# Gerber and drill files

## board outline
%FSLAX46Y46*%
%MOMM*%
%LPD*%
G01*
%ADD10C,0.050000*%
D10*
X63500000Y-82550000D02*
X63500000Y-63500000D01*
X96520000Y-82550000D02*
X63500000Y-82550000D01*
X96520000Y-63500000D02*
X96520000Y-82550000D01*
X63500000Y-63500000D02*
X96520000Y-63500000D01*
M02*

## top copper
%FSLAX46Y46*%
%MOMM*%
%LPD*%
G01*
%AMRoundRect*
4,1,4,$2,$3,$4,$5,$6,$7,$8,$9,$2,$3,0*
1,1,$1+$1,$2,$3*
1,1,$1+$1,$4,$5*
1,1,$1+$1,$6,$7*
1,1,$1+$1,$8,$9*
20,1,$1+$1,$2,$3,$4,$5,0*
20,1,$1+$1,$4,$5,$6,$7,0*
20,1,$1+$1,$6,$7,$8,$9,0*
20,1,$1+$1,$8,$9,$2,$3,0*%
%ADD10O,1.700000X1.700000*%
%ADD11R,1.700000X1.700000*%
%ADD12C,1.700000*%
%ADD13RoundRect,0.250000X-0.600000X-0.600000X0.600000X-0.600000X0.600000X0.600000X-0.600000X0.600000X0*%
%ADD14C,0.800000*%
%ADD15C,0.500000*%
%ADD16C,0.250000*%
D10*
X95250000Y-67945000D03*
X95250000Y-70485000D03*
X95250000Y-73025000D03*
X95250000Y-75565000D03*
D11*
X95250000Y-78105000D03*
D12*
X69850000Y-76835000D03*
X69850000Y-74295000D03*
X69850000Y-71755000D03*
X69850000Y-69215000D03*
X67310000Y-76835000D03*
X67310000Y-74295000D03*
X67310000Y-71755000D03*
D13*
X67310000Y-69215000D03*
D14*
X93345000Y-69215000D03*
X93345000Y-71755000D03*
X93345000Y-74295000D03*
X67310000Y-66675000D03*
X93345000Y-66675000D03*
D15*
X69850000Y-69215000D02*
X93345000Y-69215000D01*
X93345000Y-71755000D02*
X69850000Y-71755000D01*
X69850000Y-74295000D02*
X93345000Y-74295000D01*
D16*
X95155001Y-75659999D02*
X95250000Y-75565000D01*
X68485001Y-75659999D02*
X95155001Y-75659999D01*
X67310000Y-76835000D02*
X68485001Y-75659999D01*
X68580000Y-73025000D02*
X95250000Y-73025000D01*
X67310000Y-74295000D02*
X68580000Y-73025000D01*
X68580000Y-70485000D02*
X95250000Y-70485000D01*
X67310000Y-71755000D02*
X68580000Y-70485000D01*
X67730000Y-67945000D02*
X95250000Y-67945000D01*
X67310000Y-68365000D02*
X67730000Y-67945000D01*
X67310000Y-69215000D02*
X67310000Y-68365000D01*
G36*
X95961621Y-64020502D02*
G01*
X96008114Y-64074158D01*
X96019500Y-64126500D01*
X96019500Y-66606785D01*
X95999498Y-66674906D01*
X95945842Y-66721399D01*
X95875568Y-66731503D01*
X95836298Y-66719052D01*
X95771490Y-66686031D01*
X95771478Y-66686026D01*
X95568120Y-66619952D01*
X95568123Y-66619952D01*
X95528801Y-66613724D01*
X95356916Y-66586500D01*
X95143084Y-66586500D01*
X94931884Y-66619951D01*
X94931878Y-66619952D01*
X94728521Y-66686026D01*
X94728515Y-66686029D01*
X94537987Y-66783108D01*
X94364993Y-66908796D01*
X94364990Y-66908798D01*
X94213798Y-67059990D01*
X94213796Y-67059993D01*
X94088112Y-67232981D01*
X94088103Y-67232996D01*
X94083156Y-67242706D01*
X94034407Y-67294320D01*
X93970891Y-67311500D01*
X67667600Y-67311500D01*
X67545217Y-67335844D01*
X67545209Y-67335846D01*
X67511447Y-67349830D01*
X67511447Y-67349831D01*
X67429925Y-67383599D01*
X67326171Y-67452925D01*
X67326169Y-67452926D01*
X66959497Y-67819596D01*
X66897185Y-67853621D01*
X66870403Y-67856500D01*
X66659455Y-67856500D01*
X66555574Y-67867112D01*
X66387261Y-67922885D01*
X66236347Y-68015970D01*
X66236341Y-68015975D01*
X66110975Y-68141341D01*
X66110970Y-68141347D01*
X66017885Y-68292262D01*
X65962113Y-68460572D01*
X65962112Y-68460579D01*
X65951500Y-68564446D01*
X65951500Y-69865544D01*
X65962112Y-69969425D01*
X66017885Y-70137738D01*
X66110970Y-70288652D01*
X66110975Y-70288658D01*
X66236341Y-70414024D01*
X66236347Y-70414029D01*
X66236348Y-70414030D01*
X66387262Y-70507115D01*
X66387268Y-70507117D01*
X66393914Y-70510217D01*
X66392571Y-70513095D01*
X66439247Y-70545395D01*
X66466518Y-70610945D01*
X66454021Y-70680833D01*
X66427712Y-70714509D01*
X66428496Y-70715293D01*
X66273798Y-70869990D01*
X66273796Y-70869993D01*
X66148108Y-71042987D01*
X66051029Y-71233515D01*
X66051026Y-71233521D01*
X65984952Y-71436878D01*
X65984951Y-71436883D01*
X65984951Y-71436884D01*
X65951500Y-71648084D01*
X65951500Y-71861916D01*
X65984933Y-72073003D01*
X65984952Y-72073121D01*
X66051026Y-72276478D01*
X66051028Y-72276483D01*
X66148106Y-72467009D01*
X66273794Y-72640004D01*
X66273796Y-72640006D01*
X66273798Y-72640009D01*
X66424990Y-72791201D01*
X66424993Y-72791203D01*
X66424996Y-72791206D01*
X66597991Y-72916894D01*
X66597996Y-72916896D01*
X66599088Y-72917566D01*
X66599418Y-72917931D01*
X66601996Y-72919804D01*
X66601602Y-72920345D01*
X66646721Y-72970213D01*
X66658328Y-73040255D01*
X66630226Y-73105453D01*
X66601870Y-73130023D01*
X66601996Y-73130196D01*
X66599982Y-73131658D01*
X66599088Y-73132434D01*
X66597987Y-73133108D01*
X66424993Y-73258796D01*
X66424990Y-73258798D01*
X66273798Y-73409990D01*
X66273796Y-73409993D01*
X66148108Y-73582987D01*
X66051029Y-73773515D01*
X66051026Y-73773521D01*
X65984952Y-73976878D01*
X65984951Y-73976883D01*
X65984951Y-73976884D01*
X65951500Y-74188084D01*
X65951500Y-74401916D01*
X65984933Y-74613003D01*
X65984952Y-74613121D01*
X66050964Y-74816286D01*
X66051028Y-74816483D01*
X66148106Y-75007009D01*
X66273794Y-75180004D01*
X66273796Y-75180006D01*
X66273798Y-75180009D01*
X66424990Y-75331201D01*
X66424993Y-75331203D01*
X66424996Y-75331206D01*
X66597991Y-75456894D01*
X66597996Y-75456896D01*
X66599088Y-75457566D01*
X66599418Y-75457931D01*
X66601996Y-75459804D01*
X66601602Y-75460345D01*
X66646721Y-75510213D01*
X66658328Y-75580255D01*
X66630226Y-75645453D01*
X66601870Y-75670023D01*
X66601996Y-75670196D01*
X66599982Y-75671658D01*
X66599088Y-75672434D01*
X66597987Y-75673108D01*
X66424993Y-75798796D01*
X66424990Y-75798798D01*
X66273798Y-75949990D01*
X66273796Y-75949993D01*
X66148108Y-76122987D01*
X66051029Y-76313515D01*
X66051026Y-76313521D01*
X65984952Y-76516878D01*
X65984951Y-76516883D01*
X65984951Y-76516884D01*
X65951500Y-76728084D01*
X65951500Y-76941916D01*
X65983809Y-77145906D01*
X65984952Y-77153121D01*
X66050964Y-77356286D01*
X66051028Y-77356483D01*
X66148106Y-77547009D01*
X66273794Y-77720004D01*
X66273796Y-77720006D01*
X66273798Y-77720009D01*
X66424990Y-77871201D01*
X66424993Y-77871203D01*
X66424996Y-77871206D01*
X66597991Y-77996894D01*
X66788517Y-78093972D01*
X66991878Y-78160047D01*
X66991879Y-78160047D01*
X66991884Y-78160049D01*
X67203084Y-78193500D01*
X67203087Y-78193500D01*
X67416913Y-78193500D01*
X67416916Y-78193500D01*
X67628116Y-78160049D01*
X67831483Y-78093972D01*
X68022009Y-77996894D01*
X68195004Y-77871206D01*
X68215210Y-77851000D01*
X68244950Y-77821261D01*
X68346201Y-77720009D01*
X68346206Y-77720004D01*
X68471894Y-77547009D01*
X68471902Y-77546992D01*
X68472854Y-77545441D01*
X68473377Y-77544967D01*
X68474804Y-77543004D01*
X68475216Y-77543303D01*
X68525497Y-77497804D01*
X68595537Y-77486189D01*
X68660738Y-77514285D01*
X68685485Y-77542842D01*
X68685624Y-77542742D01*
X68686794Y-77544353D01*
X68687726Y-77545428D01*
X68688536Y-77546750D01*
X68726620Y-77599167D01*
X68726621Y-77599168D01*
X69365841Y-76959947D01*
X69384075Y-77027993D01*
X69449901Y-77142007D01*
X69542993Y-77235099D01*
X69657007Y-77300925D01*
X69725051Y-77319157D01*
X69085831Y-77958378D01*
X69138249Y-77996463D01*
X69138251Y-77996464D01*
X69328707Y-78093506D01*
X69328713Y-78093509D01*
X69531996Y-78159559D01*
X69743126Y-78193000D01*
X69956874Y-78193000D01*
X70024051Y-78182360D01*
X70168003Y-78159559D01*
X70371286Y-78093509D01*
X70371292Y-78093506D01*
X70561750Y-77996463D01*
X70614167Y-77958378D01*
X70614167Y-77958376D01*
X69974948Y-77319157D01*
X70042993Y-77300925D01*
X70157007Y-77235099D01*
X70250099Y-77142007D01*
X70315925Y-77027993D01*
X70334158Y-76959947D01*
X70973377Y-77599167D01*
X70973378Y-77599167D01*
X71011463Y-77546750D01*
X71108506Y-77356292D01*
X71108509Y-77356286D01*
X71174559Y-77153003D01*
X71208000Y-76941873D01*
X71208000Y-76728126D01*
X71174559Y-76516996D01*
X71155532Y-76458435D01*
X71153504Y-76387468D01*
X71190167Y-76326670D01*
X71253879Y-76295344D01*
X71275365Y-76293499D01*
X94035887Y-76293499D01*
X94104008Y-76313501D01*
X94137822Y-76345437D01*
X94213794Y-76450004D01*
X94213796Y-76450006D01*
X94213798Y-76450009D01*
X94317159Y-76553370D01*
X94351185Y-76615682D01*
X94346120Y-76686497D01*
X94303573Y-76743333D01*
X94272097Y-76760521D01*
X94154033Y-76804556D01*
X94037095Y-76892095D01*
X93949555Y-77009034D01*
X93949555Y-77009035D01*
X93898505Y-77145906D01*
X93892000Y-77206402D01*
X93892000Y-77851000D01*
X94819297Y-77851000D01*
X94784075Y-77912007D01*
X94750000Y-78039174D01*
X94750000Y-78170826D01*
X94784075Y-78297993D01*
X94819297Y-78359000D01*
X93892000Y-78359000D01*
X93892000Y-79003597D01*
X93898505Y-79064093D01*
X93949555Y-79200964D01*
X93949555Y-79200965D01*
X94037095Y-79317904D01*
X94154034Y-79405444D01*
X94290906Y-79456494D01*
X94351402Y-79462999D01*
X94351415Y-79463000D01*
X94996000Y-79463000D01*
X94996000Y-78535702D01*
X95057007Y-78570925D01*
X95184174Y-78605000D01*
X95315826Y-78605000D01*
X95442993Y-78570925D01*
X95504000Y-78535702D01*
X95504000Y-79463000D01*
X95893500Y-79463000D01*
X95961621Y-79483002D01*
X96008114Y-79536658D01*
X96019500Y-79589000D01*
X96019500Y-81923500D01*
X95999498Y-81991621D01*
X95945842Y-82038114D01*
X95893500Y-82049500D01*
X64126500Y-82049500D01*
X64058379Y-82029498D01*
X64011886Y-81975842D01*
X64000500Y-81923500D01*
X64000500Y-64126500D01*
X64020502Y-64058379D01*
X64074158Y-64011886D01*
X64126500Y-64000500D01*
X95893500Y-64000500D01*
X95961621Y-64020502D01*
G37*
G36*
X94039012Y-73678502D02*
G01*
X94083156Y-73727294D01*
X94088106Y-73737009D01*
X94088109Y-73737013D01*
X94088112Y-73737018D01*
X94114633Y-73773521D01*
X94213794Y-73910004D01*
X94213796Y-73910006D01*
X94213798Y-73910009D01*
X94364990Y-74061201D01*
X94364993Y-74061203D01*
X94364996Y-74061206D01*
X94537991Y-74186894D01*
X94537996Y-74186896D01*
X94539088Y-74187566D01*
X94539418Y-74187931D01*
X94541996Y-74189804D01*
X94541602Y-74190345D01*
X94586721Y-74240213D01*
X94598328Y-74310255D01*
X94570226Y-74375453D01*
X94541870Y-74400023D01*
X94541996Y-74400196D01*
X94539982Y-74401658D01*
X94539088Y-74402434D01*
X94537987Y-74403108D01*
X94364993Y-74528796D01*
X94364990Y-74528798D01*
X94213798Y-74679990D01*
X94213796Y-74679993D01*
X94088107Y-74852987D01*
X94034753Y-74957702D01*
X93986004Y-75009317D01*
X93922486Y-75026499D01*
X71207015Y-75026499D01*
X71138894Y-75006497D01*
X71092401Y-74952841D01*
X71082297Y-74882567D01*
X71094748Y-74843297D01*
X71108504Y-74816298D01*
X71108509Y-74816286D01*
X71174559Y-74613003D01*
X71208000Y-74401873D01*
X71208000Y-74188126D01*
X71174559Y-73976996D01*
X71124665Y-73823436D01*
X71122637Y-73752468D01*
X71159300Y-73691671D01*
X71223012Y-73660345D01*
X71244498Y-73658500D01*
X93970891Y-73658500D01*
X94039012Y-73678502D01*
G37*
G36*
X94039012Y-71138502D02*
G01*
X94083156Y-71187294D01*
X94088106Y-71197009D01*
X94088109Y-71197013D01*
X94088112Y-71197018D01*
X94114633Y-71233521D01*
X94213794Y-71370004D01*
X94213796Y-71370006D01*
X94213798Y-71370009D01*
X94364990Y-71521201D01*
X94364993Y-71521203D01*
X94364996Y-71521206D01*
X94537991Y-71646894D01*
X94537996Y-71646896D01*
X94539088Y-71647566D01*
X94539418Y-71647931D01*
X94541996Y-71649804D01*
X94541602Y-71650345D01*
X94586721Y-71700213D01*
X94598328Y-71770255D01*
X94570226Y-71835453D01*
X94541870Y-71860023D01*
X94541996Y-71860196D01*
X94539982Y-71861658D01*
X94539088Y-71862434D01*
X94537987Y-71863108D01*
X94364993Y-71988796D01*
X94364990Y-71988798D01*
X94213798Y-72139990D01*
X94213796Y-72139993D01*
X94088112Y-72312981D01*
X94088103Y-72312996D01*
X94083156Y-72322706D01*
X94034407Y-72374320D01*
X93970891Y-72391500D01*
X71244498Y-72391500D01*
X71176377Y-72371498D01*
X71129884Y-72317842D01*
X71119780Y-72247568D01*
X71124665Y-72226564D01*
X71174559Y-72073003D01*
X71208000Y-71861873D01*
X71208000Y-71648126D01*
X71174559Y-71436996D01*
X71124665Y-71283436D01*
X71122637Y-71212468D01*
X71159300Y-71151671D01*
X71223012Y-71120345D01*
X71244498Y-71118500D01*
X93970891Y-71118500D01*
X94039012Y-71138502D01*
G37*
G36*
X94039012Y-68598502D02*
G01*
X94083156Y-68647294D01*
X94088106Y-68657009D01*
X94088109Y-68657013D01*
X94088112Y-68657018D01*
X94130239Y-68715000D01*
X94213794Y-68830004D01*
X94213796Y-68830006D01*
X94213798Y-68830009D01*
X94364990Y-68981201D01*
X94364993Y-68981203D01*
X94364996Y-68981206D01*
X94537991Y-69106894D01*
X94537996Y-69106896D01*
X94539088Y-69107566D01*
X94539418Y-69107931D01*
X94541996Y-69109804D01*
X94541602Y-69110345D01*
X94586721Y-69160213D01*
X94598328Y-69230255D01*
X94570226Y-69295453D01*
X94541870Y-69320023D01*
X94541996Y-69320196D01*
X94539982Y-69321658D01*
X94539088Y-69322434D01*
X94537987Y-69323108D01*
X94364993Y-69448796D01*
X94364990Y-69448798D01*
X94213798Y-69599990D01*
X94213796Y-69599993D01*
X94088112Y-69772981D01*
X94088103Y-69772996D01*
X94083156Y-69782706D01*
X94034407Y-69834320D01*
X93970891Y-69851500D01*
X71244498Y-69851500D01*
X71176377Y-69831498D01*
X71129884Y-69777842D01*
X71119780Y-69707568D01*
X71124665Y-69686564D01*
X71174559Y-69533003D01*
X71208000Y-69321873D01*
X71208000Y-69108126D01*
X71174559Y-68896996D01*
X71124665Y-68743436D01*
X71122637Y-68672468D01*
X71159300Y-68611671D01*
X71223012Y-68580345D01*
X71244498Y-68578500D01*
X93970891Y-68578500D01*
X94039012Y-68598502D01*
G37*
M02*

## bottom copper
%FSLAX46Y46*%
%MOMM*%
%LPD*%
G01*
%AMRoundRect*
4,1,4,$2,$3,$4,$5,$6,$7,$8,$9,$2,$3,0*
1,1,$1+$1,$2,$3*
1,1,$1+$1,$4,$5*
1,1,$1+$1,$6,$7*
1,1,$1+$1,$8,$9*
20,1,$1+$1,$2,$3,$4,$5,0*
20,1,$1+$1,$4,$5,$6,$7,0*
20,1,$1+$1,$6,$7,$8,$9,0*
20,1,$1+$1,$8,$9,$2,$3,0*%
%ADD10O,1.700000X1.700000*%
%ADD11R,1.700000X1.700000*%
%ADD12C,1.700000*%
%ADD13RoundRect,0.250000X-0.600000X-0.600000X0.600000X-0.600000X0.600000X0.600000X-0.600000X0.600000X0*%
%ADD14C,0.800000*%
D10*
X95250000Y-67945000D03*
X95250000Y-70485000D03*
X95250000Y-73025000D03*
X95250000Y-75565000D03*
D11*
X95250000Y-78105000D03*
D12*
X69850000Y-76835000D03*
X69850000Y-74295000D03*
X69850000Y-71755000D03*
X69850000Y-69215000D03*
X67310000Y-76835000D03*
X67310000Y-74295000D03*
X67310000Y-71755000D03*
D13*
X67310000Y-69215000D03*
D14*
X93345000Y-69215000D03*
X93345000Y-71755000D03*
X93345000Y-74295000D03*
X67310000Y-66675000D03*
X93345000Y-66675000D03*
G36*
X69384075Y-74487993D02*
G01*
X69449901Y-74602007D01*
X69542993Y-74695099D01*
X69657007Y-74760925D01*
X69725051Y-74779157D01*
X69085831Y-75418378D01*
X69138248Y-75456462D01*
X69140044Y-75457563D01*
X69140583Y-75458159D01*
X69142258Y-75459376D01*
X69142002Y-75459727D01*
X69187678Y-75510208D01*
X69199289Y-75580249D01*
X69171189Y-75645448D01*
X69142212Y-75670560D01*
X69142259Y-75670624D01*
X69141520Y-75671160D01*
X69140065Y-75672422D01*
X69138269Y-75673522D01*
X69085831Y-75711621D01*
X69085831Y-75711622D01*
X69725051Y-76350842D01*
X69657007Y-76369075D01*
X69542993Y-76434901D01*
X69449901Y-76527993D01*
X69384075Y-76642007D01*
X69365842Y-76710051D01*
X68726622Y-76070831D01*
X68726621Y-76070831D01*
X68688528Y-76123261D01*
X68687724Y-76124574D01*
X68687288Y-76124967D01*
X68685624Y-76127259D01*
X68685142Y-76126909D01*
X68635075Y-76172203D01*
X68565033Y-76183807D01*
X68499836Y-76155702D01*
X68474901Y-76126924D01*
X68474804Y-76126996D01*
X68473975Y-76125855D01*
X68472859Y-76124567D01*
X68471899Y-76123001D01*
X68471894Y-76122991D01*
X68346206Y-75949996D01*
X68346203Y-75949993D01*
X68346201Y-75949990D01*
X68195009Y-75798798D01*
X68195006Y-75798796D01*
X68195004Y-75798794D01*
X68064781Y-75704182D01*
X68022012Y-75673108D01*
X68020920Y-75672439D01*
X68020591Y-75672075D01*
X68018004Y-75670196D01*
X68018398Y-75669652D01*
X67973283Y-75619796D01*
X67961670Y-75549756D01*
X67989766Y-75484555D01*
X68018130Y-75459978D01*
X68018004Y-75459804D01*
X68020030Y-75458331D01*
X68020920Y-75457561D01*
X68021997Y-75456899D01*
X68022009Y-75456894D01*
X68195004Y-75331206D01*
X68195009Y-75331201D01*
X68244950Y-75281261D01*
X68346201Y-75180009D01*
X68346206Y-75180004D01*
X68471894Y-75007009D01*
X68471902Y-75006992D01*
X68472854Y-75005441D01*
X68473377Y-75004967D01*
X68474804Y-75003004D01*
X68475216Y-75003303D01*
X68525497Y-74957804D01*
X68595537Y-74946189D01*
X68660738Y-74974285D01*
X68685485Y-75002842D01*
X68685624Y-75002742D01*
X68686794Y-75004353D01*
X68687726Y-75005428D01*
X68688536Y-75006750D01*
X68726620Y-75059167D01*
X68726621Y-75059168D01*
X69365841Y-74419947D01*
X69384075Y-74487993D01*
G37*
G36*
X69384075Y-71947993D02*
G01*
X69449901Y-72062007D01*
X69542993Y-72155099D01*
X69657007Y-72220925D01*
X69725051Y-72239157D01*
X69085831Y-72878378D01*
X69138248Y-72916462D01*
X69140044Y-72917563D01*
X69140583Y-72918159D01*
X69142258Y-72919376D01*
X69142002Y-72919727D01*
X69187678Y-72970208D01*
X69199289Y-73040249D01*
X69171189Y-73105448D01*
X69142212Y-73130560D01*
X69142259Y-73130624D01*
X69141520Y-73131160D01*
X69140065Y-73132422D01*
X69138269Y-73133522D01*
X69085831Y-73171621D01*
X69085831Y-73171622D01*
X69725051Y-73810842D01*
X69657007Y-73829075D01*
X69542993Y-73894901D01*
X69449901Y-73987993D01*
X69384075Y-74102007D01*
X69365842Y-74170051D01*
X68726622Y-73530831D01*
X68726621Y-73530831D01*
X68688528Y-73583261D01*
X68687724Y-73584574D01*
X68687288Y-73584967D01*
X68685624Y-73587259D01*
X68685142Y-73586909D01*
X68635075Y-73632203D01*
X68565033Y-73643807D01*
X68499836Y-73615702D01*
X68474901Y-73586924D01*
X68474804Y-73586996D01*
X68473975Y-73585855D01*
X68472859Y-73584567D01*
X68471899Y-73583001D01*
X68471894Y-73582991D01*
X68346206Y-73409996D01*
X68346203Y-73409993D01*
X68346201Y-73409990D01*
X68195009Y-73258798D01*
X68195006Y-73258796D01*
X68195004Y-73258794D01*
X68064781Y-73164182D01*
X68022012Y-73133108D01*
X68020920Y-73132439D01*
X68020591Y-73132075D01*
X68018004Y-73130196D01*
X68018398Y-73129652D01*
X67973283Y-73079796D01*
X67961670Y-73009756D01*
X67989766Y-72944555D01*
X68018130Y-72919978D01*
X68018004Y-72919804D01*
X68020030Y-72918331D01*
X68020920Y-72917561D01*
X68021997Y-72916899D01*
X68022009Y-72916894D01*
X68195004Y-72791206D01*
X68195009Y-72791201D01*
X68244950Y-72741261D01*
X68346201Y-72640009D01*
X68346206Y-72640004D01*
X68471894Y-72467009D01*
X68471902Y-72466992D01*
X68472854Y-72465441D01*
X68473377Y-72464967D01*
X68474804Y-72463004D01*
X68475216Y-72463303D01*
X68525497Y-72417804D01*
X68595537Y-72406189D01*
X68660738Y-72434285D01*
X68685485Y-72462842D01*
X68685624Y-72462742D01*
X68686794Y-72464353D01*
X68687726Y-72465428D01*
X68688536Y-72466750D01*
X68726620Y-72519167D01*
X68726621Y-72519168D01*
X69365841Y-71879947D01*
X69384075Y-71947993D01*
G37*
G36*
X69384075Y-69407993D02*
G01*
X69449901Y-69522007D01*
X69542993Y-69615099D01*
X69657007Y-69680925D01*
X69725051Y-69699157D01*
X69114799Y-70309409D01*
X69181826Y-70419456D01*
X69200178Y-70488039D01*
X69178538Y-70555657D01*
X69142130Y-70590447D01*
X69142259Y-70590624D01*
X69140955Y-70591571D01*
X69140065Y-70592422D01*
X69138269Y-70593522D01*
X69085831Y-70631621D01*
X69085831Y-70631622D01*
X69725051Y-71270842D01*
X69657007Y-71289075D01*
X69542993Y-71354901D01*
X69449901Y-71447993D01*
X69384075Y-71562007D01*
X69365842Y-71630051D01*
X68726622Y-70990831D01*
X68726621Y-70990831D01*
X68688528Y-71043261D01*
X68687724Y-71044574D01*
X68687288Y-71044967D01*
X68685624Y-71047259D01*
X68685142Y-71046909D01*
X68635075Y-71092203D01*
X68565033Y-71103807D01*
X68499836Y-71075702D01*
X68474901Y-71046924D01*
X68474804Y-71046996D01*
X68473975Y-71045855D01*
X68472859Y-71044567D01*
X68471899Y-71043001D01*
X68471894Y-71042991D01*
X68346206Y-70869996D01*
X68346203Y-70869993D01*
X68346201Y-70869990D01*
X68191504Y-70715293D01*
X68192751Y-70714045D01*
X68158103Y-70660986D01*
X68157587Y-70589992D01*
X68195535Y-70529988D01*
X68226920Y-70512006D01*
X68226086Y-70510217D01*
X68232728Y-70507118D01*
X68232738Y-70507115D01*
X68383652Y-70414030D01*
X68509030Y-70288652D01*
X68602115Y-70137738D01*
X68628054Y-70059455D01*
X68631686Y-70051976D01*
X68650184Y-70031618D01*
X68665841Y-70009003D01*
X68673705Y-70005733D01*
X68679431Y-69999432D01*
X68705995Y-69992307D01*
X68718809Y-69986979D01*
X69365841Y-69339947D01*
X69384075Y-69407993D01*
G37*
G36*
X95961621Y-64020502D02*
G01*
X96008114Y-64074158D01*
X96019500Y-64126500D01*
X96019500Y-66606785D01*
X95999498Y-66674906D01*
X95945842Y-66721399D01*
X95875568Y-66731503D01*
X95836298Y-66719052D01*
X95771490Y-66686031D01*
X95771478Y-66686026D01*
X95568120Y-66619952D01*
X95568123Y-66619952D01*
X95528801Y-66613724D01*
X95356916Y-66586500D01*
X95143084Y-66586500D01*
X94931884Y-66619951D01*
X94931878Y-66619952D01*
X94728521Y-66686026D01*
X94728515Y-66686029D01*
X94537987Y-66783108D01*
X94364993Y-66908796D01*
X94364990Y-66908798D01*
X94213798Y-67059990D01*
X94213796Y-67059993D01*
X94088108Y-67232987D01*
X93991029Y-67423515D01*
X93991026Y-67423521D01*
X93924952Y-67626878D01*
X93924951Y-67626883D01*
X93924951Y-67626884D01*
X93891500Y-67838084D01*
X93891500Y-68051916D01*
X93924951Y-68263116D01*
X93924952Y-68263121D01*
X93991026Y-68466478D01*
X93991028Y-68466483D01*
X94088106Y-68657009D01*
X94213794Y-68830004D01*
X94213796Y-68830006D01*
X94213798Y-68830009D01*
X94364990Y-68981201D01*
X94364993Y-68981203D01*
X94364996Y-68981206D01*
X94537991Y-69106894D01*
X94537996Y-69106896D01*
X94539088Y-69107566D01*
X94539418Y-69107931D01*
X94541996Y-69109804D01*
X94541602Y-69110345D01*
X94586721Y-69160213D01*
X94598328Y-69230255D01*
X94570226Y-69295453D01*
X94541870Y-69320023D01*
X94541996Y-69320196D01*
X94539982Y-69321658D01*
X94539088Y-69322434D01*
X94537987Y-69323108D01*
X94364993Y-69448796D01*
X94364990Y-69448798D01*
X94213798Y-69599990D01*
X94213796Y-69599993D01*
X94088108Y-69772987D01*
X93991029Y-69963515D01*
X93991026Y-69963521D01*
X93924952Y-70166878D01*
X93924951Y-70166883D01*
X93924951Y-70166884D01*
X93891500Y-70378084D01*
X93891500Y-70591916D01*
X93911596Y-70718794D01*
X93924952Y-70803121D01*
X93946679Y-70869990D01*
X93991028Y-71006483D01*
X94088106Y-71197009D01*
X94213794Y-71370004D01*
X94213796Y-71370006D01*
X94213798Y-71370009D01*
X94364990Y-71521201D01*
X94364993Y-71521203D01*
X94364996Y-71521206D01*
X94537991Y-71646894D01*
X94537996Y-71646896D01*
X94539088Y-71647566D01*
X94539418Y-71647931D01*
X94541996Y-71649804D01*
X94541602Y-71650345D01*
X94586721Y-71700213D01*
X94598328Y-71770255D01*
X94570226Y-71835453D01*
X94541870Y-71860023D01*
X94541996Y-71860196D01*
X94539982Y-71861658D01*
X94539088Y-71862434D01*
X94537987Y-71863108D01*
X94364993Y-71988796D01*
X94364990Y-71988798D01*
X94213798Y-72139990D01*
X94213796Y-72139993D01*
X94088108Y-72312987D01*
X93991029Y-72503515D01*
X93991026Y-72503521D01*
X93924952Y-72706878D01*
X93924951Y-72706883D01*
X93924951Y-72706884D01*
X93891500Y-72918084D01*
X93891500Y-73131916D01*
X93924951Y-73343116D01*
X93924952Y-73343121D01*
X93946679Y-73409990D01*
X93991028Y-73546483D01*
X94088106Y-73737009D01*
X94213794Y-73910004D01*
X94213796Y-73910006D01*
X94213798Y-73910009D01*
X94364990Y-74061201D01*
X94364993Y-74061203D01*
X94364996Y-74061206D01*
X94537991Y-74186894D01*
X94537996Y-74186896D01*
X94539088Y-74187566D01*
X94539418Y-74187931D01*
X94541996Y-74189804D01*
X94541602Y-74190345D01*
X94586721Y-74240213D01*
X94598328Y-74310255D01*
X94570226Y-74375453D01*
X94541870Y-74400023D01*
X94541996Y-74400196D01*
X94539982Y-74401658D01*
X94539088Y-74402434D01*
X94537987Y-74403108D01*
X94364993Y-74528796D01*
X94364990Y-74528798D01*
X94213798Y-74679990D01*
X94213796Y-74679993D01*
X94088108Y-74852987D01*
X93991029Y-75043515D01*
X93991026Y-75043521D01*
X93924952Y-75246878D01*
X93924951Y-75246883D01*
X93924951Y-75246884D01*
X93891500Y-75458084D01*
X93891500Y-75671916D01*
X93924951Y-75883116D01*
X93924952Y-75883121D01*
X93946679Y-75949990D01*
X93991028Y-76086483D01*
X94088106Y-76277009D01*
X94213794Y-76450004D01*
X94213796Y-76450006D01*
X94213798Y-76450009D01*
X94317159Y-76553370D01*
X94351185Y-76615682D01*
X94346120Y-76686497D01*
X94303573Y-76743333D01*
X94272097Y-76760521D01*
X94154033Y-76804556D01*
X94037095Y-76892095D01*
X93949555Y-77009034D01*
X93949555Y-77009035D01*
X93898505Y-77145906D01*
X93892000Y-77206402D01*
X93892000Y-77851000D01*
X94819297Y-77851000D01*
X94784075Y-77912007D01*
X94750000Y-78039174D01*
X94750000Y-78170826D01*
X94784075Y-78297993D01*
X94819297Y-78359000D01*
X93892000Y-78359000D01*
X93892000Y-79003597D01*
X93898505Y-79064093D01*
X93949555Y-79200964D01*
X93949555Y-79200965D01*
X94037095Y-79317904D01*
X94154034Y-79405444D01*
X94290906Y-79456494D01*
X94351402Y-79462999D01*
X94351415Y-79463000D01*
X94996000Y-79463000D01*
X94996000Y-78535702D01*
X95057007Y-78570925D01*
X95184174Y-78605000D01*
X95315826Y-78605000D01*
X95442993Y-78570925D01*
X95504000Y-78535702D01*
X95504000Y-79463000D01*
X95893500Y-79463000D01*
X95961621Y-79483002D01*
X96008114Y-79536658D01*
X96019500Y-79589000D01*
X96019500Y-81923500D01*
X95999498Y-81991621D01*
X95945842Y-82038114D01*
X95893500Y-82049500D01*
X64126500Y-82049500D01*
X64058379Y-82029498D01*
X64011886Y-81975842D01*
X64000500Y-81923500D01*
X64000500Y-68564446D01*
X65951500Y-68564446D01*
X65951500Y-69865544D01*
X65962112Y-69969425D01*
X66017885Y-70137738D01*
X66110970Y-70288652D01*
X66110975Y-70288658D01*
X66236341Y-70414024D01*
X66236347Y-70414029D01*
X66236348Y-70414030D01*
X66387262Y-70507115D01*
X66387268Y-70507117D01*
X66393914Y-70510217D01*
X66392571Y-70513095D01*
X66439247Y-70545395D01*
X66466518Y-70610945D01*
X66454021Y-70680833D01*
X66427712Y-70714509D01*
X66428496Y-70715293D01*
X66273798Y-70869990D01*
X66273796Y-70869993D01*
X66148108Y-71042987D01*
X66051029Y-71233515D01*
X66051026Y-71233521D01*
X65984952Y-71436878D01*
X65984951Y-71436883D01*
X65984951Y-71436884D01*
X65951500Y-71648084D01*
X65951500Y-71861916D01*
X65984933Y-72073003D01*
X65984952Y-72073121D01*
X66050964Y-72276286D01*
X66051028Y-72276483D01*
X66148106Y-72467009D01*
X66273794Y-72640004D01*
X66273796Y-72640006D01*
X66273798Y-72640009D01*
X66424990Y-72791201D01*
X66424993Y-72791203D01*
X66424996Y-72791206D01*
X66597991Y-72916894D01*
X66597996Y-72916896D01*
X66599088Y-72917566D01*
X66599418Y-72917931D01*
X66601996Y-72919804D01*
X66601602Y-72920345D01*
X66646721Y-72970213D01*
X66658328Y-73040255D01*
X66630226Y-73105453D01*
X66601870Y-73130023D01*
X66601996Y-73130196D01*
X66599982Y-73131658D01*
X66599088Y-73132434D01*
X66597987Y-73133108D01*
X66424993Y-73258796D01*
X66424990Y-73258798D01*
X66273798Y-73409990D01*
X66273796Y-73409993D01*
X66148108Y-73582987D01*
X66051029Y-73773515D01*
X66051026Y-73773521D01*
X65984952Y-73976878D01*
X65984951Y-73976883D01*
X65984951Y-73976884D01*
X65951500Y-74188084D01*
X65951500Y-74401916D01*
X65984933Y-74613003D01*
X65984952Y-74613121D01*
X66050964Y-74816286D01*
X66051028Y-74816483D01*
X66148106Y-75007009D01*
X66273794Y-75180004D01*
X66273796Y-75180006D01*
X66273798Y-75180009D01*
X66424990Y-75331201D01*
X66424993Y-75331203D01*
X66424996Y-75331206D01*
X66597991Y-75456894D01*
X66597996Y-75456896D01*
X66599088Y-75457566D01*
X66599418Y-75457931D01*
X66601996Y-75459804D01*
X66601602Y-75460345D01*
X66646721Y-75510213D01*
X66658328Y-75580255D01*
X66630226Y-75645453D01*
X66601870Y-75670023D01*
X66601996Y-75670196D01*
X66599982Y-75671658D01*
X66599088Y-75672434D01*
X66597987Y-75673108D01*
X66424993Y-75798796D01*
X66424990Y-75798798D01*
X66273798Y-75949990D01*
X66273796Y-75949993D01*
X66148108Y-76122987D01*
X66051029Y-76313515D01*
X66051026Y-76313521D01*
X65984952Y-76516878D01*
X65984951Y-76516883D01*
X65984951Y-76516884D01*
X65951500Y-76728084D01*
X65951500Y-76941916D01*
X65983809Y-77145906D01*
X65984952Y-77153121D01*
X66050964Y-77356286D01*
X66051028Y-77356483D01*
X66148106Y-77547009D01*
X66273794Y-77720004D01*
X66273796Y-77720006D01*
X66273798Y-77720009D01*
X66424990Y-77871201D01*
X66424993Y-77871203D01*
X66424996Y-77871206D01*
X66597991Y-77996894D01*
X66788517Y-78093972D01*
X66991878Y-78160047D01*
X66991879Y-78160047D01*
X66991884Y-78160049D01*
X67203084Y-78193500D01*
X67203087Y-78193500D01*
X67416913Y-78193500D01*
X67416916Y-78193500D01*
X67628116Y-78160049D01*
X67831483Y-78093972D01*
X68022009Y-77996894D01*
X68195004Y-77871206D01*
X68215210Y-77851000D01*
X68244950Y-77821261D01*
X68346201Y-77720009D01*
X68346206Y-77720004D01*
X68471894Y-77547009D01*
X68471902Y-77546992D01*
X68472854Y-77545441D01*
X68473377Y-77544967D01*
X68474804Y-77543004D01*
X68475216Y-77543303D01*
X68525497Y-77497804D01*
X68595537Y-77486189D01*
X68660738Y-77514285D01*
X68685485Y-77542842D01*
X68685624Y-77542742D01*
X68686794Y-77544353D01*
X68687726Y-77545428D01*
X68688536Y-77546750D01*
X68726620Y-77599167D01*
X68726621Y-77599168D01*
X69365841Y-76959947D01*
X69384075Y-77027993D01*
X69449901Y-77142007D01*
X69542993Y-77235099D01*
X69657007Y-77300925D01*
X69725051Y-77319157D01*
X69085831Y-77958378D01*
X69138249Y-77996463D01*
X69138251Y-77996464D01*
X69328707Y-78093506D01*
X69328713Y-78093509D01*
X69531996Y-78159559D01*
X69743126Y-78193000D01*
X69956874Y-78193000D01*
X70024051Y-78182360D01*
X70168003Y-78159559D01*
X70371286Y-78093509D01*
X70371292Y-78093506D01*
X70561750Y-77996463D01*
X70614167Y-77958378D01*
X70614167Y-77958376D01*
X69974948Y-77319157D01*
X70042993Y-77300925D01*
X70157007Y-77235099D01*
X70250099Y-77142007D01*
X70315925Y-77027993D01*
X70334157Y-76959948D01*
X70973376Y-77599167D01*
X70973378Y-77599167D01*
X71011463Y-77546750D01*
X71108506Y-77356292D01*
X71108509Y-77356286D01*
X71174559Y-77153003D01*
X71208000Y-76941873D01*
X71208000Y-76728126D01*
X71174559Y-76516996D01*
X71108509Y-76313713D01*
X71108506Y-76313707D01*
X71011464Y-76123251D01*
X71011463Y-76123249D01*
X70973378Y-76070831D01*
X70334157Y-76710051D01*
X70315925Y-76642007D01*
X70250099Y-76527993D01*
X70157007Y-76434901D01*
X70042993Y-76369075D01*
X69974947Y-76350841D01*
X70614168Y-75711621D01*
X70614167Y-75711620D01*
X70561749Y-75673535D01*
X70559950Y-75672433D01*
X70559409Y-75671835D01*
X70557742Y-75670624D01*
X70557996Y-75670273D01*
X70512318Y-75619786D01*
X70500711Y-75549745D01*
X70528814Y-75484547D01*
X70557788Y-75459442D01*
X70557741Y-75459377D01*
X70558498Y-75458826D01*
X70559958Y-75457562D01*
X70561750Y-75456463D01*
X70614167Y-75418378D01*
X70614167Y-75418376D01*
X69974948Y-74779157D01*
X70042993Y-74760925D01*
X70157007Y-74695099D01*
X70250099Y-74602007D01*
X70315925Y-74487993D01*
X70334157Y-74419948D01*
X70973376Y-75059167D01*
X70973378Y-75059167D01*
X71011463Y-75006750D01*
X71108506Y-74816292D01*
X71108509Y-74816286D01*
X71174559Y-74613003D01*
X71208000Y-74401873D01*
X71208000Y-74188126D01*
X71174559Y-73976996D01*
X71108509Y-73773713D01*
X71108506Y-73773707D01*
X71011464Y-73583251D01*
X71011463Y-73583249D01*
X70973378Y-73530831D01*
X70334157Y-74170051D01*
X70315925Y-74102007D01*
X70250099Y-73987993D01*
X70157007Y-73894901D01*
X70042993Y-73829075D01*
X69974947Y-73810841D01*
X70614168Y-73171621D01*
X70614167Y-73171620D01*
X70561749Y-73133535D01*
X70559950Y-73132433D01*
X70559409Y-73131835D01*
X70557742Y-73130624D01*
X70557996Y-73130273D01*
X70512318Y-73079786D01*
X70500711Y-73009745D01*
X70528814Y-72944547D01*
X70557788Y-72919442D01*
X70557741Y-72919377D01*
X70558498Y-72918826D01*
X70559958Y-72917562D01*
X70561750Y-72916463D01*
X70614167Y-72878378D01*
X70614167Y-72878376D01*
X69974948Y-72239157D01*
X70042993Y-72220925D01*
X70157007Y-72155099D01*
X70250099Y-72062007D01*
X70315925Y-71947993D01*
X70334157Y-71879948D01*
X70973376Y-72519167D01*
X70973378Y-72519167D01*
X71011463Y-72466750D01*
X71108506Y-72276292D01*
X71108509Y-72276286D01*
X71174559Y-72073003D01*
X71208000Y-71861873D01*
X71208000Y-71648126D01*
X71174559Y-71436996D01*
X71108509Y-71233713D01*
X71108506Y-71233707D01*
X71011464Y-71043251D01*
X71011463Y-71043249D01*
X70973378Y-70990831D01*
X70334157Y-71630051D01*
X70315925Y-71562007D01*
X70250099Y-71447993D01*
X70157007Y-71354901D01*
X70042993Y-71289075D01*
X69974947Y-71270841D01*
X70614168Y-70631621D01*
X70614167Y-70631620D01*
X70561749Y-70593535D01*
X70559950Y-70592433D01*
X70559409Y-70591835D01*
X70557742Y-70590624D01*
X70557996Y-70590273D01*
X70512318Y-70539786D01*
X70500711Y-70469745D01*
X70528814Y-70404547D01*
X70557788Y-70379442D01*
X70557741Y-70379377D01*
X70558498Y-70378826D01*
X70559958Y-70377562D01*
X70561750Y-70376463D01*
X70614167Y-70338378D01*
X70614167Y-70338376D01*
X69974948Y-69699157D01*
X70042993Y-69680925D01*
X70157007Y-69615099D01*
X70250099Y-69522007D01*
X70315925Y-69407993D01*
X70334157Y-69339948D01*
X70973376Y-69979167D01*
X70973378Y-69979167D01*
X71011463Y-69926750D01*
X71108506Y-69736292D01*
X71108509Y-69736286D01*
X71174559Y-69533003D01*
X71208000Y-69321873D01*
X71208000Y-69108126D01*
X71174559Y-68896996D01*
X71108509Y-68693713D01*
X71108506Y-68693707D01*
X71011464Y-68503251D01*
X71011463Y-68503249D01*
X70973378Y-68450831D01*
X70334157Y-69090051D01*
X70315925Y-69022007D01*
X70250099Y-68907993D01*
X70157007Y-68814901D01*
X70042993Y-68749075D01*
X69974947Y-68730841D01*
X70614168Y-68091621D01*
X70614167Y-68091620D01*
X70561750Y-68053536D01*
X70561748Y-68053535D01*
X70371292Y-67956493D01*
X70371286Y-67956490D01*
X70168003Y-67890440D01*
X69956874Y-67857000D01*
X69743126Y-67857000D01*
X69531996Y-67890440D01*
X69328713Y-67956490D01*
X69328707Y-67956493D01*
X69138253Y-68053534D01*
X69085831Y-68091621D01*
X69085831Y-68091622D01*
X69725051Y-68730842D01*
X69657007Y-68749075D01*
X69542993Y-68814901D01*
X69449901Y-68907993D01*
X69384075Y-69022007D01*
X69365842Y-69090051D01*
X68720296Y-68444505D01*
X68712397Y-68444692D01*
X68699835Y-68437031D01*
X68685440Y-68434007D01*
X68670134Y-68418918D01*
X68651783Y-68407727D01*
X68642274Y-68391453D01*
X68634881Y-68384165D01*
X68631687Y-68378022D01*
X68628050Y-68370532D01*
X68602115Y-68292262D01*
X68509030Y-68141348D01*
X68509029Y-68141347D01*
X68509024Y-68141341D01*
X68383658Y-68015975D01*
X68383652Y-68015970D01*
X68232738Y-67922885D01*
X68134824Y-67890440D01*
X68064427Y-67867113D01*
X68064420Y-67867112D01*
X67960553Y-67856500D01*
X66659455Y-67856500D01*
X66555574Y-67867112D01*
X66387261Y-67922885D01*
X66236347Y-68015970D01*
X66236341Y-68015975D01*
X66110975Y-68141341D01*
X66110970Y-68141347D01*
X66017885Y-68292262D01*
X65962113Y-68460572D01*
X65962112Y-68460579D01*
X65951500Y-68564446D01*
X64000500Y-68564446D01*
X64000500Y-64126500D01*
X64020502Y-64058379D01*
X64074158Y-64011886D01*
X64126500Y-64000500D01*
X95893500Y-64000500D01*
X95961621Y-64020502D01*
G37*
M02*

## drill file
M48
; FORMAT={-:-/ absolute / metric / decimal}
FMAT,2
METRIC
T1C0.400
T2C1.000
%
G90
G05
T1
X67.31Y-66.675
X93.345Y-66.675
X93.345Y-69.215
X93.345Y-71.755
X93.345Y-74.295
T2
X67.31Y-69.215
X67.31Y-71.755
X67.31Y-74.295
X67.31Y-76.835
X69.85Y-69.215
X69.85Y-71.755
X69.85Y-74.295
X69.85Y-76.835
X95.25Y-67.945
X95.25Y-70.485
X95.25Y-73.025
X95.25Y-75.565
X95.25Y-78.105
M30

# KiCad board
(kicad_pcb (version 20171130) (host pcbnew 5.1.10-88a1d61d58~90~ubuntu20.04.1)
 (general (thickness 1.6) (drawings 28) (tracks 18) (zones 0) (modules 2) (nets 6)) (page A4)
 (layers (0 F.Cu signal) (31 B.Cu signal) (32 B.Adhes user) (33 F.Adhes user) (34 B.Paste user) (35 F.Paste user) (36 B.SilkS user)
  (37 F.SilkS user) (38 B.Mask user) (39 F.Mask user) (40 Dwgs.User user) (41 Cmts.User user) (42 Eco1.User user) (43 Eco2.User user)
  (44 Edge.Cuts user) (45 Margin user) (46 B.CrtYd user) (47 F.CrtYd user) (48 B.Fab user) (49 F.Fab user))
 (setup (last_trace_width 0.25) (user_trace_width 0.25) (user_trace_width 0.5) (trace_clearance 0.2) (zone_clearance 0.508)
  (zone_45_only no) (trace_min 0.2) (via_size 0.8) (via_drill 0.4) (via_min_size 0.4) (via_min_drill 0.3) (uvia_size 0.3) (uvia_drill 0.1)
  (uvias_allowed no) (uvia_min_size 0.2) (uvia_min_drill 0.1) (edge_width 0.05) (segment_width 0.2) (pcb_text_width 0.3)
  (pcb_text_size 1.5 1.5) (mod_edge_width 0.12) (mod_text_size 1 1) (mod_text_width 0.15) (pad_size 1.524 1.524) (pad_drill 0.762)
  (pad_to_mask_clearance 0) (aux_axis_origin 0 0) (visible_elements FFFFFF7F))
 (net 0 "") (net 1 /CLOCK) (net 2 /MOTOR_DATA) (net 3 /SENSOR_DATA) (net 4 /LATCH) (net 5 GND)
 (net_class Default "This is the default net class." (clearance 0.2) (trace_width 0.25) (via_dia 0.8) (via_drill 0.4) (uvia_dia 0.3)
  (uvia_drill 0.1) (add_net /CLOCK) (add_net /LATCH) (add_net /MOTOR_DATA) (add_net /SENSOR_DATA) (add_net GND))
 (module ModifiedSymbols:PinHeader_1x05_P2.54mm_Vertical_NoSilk (layer B.Cu) (at 95.25 78.105)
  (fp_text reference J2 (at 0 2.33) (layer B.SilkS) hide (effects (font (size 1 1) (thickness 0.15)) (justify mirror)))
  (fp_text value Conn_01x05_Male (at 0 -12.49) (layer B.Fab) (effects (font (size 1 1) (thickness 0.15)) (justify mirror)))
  (pad 5 thru_hole oval (at 0 -10.16) (size 1.7 1.7) (drill 1) (layers *.Cu *.Mask) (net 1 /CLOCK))
  (pad 4 thru_hole oval (at 0 -7.62) (size 1.7 1.7) (drill 1) (layers *.Cu *.Mask) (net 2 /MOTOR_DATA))
  (pad 3 thru_hole oval (at 0 -5.08) (size 1.7 1.7) (drill 1) (layers *.Cu *.Mask) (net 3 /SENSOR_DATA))
  (pad 2 thru_hole oval (at 0 -2.54) (size 1.7 1.7) (drill 1) (layers *.Cu *.Mask) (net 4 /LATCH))
  (pad 1 thru_hole rect (at 0 0) (size 1.7 1.7) (drill 1) (layers *.Cu *.Mask) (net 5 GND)))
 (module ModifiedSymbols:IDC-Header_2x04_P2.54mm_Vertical (layer F.Cu) (at 67.31 69.215)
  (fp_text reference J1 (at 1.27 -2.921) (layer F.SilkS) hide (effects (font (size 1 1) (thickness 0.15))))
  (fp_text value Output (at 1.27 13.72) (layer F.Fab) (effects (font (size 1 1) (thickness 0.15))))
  (pad 8 thru_hole circle (at 2.54 7.62) (size 1.7 1.7) (drill 1) (layers *.Cu *.Mask) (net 5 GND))
  (pad 6 thru_hole circle (at 2.54 5.08) (size 1.7 1.7) (drill 1) (layers *.Cu *.Mask) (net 5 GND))
  (pad 4 thru_hole circle (at 2.54 2.54) (size 1.7 1.7) (drill 1) (layers *.Cu *.Mask) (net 5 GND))
  (pad 2 thru_hole circle (at 2.54 0) (size 1.7 1.7) (drill 1) (layers *.Cu *.Mask) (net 5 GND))
  (pad 7 thru_hole circle (at 0 7.62) (size 1.7 1.7) (drill 1) (layers *.Cu *.Mask) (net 4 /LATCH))
  (pad 5 thru_hole circle (at 0 5.08) (size 1.7 1.7) (drill 1) (layers *.Cu *.Mask) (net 3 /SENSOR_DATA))
  (pad 3 thru_hole circle (at 0 2.54) (size 1.7 1.7) (drill 1) (layers *.Cu *.Mask) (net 2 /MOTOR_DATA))
  (pad 1 thru_hole roundrect (at 0 0) (size 1.7 1.7) (drill 1) (layers *.Cu *.Mask) (roundrect_rratio 0.147059) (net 1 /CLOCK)))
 (gr_line (start 63.5 82.55) (end 63.5 63.5) (layer Edge.Cuts) (width 0.05))
 (gr_line (start 96.52 82.55) (end 63.5 82.55) (layer Edge.Cuts) (width 0.05))
 (gr_line (start 96.52 63.5) (end 96.52 82.55) (layer Edge.Cuts) (width 0.05))
 (gr_line (start 63.5 63.5) (end 96.52 63.5) (layer Edge.Cuts) (width 0.05))
 (via (at 93.345 69.215) (size 0.8) (drill 0.4) (layers F.Cu B.Cu) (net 5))
 (via (at 93.345 71.755) (size 0.8) (drill 0.4) (layers F.Cu B.Cu) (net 5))
 (via (at 93.345 74.295) (size 0.8) (drill 0.4) (layers F.Cu B.Cu) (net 5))
 (segment (start 69.85 69.215) (end 93.345 69.215) (width 0.5) (layer F.Cu) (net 5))
 (segment (start 93.345 71.755) (end 69.85 71.755) (width 0.5) (layer F.Cu) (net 5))
 (segment (start 69.85 74.295) (end 93.345 74.295) (width 0.5) (layer F.Cu) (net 5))
 (via (at 67.31 66.675) (size 0.8) (drill 0.4) (layers F.Cu B.Cu) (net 5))
 (via (at 93.345 66.675) (size 0.8) (drill 0.4) (layers F.Cu B.Cu) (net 5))
 (segment (start 95.155001 75.659999) (end 95.25 75.565) (width 0.25) (layer F.Cu) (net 4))
 (segment (start 68.485001 75.659999) (end 95.155001 75.659999) (width 0.25) (layer F.Cu) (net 4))
 (segment (start 67.31 76.835) (end 68.485001 75.659999) (width 0.25) (layer F.Cu) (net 4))
 (segment (start 68.58 73.025) (end 95.25 73.025) (width 0.25) (layer F.Cu) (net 3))
 (segment (start 67.31 74.295) (end 68.58 73.025) (width 0.25) (layer F.Cu) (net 3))
 (segment (start 68.58 70.485) (end 95.25 70.485) (width 0.25) (layer F.Cu) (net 2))
 (segment (start 67.31 71.755) (end 68.58 70.485) (width 0.25) (layer F.Cu) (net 2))
 (segment (start 67.73 67.945) (end 95.25 67.945) (width 0.25) (layer F.Cu) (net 1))
 (segment (start 67.31 68.365) (end 67.73 67.945) (width 0.25) (layer F.Cu) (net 1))
 (segment (start 67.31 69.215) (end 67.31 68.365) (width 0.25) (layer F.Cu) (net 1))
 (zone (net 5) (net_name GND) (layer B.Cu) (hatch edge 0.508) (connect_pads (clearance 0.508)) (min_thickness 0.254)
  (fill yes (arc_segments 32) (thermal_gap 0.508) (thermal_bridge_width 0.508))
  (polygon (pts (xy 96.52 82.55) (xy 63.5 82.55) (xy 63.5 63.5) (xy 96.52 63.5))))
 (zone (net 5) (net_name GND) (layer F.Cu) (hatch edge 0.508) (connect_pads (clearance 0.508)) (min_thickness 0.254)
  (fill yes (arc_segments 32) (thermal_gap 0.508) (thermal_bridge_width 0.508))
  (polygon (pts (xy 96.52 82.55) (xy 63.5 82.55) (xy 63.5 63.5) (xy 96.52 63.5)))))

